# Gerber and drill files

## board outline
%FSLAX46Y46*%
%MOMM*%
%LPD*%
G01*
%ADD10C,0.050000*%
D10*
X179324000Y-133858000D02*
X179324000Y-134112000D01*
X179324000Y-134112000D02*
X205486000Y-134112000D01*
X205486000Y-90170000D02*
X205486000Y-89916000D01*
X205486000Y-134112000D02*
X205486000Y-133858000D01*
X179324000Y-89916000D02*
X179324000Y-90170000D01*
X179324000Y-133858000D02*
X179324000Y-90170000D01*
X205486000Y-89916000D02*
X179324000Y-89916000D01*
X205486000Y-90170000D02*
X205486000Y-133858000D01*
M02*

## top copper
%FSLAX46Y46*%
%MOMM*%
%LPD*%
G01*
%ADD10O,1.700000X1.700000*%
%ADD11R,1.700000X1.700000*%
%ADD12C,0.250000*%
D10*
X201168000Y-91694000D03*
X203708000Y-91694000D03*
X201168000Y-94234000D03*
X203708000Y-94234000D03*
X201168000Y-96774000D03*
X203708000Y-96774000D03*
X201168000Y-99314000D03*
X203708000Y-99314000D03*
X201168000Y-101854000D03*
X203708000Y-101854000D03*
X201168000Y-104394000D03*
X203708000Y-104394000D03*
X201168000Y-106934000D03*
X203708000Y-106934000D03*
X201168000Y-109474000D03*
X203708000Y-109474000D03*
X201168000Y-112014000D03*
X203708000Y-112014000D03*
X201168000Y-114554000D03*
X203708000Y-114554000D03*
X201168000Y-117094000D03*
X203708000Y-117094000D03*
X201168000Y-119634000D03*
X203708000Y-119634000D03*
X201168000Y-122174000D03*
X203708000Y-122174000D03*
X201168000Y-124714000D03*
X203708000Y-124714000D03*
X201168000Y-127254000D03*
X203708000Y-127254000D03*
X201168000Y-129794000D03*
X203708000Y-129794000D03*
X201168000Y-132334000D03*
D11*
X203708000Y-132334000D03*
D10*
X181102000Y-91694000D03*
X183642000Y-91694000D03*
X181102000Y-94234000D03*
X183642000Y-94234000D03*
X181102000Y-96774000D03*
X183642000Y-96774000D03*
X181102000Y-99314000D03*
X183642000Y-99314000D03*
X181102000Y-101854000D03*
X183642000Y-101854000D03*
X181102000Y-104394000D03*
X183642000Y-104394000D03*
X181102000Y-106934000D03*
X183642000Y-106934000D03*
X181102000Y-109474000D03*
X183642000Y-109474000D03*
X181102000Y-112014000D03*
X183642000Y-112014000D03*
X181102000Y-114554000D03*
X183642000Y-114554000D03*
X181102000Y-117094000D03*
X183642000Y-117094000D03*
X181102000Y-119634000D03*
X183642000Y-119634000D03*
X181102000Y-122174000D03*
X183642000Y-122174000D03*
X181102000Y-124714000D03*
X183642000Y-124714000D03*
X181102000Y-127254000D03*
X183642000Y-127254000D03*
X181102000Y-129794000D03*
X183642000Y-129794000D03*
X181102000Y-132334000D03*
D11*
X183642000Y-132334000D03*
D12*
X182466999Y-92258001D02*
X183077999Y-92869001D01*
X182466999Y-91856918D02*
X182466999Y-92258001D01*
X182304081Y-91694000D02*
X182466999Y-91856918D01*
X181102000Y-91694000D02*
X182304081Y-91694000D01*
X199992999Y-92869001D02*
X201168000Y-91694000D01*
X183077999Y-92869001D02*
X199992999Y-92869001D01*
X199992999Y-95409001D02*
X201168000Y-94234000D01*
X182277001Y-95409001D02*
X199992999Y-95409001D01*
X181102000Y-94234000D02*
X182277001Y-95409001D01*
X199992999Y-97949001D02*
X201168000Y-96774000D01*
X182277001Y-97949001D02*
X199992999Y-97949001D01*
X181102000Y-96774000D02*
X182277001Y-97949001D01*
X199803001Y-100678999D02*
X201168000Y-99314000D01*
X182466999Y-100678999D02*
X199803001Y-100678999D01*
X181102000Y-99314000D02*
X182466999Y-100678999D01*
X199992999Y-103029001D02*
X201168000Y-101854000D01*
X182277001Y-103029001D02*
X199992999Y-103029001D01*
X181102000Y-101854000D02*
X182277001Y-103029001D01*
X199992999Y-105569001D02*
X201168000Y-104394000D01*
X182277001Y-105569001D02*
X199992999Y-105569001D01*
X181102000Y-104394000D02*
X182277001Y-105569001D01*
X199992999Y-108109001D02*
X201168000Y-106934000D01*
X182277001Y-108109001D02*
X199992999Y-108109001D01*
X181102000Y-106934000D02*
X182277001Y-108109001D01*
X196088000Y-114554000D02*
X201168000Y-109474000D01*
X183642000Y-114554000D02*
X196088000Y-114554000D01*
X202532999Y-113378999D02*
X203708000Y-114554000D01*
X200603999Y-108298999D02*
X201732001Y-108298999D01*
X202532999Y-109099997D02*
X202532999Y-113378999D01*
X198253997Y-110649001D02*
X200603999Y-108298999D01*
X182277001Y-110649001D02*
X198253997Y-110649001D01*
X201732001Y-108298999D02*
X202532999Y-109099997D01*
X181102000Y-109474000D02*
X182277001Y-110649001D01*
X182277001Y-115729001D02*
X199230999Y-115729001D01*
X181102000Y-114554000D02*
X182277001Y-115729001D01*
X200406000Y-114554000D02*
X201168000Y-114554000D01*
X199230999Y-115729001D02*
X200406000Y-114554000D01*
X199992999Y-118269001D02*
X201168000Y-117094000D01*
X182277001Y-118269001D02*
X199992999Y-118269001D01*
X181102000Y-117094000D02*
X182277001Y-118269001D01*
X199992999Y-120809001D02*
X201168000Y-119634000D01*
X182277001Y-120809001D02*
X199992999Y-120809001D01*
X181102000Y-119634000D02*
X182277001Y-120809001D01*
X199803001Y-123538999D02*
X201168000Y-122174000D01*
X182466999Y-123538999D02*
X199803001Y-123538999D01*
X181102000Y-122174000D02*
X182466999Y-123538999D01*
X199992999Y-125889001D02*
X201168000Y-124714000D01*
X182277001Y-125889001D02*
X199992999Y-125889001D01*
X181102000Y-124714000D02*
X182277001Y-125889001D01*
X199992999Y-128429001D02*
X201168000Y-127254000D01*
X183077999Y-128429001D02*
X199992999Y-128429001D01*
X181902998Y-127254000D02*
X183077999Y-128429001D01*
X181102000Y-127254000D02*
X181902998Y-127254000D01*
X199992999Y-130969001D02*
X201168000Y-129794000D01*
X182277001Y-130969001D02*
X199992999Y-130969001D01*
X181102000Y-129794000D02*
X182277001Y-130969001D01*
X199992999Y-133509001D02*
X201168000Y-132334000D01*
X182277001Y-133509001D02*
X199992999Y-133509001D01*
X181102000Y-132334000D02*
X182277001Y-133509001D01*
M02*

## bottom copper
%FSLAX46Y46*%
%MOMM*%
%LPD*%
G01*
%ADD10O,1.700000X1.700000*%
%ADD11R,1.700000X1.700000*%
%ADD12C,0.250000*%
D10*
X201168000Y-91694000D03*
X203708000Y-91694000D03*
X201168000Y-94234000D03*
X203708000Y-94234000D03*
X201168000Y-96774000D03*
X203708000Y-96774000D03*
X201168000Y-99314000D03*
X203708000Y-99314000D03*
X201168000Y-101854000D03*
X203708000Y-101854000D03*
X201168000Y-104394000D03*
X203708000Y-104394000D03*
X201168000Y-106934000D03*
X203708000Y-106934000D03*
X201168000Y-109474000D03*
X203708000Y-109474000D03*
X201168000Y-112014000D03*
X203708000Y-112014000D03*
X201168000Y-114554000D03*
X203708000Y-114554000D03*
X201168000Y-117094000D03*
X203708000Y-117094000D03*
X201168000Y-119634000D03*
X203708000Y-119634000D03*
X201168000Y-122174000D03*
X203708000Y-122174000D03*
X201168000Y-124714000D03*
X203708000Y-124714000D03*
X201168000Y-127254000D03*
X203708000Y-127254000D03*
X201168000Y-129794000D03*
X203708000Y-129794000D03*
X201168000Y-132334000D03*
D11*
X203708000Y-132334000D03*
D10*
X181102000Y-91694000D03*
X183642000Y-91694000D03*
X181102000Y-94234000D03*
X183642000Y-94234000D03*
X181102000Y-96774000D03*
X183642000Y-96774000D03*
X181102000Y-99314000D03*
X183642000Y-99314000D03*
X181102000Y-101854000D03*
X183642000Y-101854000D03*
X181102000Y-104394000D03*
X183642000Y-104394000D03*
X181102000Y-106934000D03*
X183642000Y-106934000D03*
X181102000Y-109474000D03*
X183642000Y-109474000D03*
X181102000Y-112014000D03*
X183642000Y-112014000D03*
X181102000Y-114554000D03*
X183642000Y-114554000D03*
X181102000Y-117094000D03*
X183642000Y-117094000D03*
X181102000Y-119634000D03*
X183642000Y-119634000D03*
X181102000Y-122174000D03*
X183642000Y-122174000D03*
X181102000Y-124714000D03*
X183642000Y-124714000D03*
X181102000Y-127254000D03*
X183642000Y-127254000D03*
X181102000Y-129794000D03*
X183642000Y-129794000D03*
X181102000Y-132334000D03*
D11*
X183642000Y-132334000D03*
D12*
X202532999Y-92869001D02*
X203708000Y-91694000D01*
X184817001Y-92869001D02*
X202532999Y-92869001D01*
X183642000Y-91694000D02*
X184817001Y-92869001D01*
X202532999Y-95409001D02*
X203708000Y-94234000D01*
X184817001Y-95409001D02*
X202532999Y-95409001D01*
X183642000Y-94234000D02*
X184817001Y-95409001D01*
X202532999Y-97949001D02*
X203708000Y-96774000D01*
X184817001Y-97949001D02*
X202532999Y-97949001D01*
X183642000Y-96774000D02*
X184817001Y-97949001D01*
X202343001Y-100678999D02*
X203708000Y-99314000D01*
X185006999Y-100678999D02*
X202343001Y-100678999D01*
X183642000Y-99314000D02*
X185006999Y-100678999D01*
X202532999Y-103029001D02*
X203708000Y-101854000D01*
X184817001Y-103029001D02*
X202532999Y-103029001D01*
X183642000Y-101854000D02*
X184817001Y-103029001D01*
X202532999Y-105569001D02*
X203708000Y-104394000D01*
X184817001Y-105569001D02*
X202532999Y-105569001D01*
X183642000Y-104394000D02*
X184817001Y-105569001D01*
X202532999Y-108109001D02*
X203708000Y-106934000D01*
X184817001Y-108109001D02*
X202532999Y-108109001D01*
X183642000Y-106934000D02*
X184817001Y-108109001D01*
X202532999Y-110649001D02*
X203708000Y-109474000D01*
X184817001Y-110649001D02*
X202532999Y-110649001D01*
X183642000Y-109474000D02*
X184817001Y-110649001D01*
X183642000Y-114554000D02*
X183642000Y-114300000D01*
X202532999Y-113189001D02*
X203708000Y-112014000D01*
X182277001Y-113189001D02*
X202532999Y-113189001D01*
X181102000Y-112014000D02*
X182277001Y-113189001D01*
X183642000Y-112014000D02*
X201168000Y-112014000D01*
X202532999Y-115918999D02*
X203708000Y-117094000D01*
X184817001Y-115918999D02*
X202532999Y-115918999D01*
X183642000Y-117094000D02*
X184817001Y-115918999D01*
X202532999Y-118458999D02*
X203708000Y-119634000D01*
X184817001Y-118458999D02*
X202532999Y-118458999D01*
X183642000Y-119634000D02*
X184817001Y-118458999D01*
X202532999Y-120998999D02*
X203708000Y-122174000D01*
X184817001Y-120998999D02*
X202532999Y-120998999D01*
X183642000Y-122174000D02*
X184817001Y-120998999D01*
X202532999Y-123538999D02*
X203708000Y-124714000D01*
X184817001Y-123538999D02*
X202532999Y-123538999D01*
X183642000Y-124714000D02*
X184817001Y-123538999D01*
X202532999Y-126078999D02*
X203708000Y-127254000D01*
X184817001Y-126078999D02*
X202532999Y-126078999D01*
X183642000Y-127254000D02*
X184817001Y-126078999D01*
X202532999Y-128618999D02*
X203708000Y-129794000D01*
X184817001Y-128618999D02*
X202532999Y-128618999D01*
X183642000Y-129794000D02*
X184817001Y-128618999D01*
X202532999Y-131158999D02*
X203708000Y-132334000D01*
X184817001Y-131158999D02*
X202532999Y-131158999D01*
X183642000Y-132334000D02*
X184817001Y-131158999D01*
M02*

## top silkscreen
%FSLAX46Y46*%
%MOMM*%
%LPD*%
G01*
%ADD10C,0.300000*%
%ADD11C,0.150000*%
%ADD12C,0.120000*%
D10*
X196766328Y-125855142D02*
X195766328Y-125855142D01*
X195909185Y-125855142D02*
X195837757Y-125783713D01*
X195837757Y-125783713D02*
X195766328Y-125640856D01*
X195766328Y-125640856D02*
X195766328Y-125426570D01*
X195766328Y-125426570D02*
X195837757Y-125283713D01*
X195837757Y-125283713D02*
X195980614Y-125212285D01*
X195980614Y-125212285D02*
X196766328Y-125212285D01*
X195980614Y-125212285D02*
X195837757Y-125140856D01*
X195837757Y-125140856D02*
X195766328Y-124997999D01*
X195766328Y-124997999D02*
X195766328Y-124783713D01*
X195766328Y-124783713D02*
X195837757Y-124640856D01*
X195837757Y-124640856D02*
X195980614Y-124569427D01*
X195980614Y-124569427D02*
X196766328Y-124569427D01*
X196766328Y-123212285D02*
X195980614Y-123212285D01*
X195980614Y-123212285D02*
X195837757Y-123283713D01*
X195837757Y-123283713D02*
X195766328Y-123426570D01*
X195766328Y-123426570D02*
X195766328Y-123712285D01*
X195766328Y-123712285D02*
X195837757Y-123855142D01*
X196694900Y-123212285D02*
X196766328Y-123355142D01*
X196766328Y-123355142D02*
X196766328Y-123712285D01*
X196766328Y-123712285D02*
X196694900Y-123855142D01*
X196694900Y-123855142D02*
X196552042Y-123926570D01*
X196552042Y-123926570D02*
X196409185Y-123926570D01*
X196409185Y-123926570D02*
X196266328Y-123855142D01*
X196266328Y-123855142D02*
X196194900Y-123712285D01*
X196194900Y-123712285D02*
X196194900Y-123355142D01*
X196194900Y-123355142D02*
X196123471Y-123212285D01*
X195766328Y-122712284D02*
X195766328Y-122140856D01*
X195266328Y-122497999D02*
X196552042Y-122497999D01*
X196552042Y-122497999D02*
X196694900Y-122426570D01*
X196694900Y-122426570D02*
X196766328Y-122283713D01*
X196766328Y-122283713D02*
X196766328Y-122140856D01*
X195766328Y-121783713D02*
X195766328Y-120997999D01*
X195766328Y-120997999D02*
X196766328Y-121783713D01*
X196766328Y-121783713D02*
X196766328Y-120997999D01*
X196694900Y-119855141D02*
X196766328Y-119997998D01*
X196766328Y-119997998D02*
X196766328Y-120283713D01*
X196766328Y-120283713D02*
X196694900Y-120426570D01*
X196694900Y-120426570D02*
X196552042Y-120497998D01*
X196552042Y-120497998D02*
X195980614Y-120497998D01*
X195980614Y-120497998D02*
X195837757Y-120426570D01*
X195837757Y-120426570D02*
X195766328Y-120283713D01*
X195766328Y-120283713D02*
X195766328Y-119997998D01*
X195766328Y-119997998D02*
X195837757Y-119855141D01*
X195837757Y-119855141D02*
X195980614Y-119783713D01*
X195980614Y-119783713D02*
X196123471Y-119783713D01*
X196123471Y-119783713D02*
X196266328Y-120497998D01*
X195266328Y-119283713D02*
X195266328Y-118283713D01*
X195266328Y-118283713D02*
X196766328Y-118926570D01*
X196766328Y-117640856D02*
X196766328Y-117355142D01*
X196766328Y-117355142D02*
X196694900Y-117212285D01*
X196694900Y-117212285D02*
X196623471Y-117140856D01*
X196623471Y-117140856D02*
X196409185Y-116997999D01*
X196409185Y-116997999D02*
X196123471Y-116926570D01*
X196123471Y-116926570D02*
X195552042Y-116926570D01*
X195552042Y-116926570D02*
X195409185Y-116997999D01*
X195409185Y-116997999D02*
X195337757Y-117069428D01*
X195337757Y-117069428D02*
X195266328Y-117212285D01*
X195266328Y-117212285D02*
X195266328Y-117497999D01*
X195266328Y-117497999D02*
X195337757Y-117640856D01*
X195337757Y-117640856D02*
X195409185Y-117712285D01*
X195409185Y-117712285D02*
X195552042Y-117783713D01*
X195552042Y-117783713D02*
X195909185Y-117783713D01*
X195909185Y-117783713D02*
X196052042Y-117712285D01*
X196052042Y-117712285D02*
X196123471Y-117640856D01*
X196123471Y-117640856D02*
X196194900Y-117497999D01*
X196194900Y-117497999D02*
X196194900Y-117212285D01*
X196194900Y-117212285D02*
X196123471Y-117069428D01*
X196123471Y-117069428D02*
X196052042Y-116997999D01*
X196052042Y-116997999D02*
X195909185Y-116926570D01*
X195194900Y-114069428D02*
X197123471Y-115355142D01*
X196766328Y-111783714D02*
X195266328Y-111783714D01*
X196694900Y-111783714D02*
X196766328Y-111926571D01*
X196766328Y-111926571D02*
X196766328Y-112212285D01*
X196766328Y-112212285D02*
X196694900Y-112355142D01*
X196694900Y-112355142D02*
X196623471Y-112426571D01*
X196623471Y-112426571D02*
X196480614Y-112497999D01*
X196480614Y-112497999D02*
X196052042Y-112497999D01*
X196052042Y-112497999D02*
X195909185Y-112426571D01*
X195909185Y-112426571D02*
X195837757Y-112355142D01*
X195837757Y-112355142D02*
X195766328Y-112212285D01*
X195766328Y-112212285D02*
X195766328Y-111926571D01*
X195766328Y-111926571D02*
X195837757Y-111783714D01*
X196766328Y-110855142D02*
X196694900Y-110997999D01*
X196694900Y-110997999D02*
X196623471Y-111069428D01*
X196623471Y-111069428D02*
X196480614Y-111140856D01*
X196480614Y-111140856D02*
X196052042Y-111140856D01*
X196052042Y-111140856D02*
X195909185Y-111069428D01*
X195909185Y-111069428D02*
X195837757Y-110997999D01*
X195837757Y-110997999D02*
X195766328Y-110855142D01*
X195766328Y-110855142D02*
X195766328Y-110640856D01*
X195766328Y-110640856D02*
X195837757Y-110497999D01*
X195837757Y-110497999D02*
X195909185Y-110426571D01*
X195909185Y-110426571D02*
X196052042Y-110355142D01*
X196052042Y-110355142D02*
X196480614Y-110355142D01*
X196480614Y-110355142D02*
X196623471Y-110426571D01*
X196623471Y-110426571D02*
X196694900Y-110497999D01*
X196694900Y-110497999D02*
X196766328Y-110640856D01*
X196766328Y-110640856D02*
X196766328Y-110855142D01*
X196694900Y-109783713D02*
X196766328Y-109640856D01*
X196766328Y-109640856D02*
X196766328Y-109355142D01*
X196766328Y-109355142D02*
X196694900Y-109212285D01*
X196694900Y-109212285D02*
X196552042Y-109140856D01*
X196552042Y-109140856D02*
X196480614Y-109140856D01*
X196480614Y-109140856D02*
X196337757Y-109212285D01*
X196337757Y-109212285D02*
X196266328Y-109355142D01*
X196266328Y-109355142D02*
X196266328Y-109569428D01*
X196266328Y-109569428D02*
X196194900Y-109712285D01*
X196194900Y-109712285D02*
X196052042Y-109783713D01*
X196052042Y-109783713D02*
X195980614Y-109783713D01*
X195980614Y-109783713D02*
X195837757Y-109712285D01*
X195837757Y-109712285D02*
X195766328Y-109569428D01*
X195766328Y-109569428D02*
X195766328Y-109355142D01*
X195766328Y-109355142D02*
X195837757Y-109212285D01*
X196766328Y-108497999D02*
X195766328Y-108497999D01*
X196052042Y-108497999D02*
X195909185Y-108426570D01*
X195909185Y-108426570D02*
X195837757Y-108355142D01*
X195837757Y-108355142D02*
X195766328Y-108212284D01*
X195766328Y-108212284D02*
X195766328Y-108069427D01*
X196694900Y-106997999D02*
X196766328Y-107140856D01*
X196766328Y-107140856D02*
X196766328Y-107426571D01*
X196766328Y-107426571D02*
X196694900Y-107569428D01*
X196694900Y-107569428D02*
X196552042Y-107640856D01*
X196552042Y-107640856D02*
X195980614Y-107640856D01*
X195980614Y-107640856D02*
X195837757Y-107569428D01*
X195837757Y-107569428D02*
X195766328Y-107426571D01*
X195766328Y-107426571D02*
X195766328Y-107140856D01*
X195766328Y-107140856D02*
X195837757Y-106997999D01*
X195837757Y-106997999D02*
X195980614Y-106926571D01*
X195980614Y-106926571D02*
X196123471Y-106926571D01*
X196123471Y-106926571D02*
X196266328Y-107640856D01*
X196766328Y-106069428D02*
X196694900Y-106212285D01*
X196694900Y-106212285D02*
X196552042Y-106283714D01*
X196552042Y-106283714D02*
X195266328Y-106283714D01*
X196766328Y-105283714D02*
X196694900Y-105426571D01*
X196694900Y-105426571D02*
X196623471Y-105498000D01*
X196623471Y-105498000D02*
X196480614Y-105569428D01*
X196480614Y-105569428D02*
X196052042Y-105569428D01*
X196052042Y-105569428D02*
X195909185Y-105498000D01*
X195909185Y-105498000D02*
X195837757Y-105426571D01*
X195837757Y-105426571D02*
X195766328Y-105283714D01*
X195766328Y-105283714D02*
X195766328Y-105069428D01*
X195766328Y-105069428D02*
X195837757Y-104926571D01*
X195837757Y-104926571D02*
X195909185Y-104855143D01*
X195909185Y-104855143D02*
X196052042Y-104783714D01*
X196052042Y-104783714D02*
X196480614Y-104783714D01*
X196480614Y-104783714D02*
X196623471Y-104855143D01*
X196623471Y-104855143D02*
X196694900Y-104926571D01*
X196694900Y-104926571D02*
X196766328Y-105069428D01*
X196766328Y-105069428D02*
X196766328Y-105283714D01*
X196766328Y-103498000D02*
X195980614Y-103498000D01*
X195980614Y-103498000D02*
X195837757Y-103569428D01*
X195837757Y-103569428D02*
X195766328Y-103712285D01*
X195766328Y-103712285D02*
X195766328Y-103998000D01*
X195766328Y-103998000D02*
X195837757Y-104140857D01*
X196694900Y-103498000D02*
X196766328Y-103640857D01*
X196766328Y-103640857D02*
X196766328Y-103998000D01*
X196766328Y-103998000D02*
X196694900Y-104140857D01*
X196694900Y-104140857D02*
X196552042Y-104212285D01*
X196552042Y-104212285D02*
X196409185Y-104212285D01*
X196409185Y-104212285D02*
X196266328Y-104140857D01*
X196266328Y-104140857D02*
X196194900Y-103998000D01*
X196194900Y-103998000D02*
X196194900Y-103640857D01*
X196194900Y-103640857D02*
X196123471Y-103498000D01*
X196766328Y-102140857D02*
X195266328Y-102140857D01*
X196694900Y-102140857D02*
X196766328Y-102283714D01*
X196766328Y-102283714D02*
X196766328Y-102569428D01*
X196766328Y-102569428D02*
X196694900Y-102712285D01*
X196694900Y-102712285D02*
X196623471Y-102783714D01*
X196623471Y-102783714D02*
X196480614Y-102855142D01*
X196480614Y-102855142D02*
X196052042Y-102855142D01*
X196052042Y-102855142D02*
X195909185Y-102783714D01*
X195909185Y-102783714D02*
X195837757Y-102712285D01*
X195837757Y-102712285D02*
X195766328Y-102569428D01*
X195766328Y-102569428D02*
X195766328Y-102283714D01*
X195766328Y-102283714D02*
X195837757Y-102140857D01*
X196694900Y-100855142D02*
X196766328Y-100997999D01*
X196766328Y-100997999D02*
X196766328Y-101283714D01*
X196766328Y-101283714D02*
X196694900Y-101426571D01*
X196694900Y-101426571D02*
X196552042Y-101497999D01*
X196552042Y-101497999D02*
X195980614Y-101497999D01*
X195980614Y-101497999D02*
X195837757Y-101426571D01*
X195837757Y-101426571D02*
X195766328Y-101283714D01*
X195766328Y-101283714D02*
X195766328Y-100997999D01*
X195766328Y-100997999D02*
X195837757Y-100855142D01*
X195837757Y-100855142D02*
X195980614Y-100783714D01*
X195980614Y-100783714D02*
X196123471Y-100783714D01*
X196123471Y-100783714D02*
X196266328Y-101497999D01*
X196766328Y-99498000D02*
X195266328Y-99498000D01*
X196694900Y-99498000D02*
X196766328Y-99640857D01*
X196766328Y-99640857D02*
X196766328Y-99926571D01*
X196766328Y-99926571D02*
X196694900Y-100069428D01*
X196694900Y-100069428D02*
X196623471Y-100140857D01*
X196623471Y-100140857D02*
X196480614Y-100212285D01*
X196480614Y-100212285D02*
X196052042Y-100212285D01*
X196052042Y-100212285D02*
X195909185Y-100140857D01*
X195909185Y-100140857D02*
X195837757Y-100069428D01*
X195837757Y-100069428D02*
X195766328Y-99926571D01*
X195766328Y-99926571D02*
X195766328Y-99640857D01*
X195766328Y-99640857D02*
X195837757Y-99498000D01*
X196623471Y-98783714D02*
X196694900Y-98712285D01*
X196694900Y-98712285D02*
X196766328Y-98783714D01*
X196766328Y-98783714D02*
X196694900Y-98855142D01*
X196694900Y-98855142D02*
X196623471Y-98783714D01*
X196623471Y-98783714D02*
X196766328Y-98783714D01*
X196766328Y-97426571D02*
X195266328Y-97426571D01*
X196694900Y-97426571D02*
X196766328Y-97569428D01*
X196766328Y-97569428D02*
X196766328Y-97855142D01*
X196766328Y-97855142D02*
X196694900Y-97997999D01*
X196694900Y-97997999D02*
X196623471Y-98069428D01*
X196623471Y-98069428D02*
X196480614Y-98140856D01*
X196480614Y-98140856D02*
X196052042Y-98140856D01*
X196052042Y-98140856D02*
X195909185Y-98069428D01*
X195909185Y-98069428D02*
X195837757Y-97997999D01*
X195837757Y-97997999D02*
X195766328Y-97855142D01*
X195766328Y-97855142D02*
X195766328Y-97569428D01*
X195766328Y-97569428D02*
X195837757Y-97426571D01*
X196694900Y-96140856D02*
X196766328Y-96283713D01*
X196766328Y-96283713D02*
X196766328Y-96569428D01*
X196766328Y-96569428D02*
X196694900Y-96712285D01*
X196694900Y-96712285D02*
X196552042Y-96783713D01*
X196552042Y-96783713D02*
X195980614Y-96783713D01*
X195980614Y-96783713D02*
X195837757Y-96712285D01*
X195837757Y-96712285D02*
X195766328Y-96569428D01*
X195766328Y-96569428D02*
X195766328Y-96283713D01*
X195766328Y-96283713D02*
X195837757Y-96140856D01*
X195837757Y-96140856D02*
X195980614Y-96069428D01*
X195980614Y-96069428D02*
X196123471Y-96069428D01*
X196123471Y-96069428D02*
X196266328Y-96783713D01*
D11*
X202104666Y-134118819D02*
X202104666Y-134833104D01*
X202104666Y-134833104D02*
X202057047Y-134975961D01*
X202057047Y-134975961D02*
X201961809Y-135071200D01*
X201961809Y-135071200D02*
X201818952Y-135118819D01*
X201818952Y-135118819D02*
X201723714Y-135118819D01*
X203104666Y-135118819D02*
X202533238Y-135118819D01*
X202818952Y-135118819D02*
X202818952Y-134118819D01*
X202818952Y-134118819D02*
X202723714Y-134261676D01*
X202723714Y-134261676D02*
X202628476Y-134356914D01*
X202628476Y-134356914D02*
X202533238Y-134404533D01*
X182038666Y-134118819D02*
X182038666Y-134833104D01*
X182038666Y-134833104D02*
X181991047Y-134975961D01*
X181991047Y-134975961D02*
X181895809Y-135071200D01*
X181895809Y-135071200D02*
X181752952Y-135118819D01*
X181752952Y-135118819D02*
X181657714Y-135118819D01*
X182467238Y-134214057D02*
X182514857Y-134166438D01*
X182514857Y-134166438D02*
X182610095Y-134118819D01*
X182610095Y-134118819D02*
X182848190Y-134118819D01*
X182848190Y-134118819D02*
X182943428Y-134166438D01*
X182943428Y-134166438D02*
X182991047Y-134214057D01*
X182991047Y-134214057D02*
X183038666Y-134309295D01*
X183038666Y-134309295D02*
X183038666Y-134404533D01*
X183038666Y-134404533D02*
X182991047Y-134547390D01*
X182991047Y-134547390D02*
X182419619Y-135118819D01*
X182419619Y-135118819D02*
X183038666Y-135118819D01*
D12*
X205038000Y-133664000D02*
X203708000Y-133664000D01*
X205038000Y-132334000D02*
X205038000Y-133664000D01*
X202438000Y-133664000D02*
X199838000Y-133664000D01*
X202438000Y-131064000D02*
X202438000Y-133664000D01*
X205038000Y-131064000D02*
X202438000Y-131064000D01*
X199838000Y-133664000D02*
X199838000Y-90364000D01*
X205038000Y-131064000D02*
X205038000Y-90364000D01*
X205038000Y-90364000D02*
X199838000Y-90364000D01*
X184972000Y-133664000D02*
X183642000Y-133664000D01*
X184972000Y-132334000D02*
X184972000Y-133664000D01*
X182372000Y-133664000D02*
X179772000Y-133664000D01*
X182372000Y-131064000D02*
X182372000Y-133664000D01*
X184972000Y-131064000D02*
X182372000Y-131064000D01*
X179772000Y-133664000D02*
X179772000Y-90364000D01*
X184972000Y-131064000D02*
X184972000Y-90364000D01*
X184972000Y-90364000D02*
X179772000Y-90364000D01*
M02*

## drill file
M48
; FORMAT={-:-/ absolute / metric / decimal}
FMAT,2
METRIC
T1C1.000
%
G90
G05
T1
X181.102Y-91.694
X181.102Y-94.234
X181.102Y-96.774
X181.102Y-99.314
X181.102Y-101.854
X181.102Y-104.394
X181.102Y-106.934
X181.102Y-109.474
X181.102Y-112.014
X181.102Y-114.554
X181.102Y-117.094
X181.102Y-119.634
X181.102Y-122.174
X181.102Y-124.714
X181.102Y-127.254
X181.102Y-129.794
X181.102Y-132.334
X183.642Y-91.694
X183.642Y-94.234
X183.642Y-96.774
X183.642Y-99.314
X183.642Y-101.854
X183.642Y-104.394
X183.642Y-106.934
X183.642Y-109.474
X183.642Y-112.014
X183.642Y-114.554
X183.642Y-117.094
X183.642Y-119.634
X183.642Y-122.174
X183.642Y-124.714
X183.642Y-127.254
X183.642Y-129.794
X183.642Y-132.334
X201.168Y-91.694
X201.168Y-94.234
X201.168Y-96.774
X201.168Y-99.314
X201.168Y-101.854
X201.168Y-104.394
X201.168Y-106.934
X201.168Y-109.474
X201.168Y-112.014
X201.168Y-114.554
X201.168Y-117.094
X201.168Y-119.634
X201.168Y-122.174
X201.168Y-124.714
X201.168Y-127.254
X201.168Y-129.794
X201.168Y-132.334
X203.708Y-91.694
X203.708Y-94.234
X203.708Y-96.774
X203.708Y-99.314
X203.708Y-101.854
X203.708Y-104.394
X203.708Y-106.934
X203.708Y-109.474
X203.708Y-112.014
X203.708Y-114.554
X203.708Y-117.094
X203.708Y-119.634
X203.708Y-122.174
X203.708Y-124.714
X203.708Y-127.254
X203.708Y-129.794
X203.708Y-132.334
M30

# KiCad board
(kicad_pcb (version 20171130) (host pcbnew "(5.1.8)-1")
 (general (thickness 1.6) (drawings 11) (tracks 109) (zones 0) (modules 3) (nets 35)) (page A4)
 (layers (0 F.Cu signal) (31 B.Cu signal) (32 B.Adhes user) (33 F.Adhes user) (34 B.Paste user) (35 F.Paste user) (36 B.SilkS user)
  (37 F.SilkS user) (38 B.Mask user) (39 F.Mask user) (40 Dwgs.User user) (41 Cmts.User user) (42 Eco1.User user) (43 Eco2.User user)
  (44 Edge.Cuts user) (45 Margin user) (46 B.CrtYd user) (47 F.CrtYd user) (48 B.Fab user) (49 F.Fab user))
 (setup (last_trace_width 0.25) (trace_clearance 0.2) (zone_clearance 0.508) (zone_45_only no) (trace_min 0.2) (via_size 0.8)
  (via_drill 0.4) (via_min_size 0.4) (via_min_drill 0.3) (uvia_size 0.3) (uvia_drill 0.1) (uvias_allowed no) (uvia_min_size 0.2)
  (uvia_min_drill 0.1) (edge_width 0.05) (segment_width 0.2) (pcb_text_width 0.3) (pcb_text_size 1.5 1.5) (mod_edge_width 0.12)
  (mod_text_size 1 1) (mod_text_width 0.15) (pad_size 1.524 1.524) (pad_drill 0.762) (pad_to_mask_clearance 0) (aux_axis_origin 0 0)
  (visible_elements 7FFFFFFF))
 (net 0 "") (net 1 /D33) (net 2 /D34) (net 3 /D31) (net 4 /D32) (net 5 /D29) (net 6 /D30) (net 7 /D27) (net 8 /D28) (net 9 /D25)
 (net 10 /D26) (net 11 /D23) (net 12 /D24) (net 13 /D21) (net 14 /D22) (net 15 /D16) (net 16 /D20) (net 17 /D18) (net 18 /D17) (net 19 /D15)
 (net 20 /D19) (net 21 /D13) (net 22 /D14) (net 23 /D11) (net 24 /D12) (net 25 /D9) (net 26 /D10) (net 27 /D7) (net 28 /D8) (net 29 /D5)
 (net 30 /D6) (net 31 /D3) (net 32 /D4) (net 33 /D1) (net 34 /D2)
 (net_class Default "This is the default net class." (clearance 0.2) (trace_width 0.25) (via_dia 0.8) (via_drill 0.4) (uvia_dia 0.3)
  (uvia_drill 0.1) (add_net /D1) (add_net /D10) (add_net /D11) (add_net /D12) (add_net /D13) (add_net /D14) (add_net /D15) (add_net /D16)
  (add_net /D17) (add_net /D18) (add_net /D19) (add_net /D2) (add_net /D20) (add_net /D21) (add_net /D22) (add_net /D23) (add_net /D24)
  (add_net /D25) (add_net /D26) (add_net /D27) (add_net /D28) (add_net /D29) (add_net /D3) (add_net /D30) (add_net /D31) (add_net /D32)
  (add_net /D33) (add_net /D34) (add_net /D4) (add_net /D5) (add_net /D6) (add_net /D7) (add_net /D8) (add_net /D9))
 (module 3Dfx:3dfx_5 (layer B.Cu) (at 193.294 112.776 270)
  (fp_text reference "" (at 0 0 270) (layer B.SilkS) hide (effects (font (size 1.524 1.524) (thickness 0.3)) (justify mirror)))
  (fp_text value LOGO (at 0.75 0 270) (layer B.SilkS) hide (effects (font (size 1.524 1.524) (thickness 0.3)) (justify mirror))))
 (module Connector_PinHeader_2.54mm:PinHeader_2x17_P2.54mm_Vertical (layer F.Cu) (at 203.708 132.334 180)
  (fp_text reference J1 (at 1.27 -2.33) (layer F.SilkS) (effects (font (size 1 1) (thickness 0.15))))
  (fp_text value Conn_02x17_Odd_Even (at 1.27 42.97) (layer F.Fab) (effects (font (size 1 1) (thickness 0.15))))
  (fp_line (start -1.33 -1.33) (end 0 -1.33) (layer F.SilkS) (width 0.12))
  (fp_line (start -1.33 0) (end -1.33 -1.33) (layer F.SilkS) (width 0.12))
  (fp_line (start 1.27 -1.33) (end 3.87 -1.33) (layer F.SilkS) (width 0.12))
  (fp_line (start 1.27 1.27) (end 1.27 -1.33) (layer F.SilkS) (width 0.12))
  (fp_line (start -1.33 1.27) (end 1.27 1.27) (layer F.SilkS) (width 0.12))
  (fp_line (start 3.87 -1.33) (end 3.87 41.97) (layer F.SilkS) (width 0.12))
  (fp_line (start -1.33 1.27) (end -1.33 41.97) (layer F.SilkS) (width 0.12))
  (fp_line (start -1.33 41.97) (end 3.87 41.97) (layer F.SilkS) (width 0.12))
  (pad 34 thru_hole oval (at 2.54 40.64 180) (size 1.7 1.7) (drill 1) (layers *.Cu *.Mask) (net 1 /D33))
  (pad 33 thru_hole oval (at 0 40.64 180) (size 1.7 1.7) (drill 1) (layers *.Cu *.Mask) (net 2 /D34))
  (pad 32 thru_hole oval (at 2.54 38.1 180) (size 1.7 1.7) (drill 1) (layers *.Cu *.Mask) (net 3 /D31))
  (pad 31 thru_hole oval (at 0 38.1 180) (size 1.7 1.7) (drill 1) (layers *.Cu *.Mask) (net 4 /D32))
  (pad 30 thru_hole oval (at 2.54 35.56 180) (size 1.7 1.7) (drill 1) (layers *.Cu *.Mask) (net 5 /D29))
  (pad 29 thru_hole oval (at 0 35.56 180) (size 1.7 1.7) (drill 1) (layers *.Cu *.Mask) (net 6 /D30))
  (pad 28 thru_hole oval (at 2.54 33.02 180) (size 1.7 1.7) (drill 1) (layers *.Cu *.Mask) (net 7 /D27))
  (pad 27 thru_hole oval (at 0 33.02 180) (size 1.7 1.7) (drill 1) (layers *.Cu *.Mask) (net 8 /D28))
  (pad 26 thru_hole oval (at 2.54 30.48 180) (size 1.7 1.7) (drill 1) (layers *.Cu *.Mask) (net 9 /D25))
  (pad 25 thru_hole oval (at 0 30.48 180) (size 1.7 1.7) (drill 1) (layers *.Cu *.Mask) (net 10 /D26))
  (pad 24 thru_hole oval (at 2.54 27.94 180) (size 1.7 1.7) (drill 1) (layers *.Cu *.Mask) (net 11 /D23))
  (pad 23 thru_hole oval (at 0 27.94 180) (size 1.7 1.7) (drill 1) (layers *.Cu *.Mask) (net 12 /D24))
  (pad 22 thru_hole oval (at 2.54 25.4 180) (size 1.7 1.7) (drill 1) (layers *.Cu *.Mask) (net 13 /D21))
  (pad 21 thru_hole oval (at 0 25.4 180) (size 1.7 1.7) (drill 1) (layers *.Cu *.Mask) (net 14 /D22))
  (pad 20 thru_hole oval (at 2.54 22.86 180) (size 1.7 1.7) (drill 1) (layers *.Cu *.Mask) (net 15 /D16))
  (pad 19 thru_hole oval (at 0 22.86 180) (size 1.7 1.7) (drill 1) (layers *.Cu *.Mask) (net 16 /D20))
  (pad 18 thru_hole oval (at 2.54 20.32 180) (size 1.7 1.7) (drill 1) (layers *.Cu *.Mask) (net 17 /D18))
  (pad 17 thru_hole oval (at 0 20.32 180) (size 1.7 1.7) (drill 1) (layers *.Cu *.Mask) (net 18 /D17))
  (pad 16 thru_hole oval (at 2.54 17.78 180) (size 1.7 1.7) (drill 1) (layers *.Cu *.Mask) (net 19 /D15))
  (pad 15 thru_hole oval (at 0 17.78 180) (size 1.7 1.7) (drill 1) (layers *.Cu *.Mask) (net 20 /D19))
  (pad 14 thru_hole oval (at 2.54 15.24 180) (size 1.7 1.7) (drill 1) (layers *.Cu *.Mask) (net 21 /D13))
  (pad 13 thru_hole oval (at 0 15.24 180) (size 1.7 1.7) (drill 1) (layers *.Cu *.Mask) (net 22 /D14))
  (pad 12 thru_hole oval (at 2.54 12.7 180) (size 1.7 1.7) (drill 1) (layers *.Cu *.Mask) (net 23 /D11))
  (pad 11 thru_hole oval (at 0 12.7 180) (size 1.7 1.7) (drill 1) (layers *.Cu *.Mask) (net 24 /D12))
  (pad 10 thru_hole oval (at 2.54 10.16 180) (size 1.7 1.7) (drill 1) (layers *.Cu *.Mask) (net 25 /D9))
  (pad 9 thru_hole oval (at 0 10.16 180) (size 1.7 1.7) (drill 1) (layers *.Cu *.Mask) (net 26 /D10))
  (pad 8 thru_hole oval (at 2.54 7.62 180) (size 1.7 1.7) (drill 1) (layers *.Cu *.Mask) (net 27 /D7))
  (pad 7 thru_hole oval (at 0 7.62 180) (size 1.7 1.7) (drill 1) (layers *.Cu *.Mask) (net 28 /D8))
  (pad 6 thru_hole oval (at 2.54 5.08 180) (size 1.7 1.7) (drill 1) (layers *.Cu *.Mask) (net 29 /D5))
  (pad 5 thru_hole oval (at 0 5.08 180) (size 1.7 1.7) (drill 1) (layers *.Cu *.Mask) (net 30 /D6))
  (pad 4 thru_hole oval (at 2.54 2.54 180) (size 1.7 1.7) (drill 1) (layers *.Cu *.Mask) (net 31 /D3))
  (pad 3 thru_hole oval (at 0 2.54 180) (size 1.7 1.7) (drill 1) (layers *.Cu *.Mask) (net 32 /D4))
  (pad 2 thru_hole oval (at 2.54 0 180) (size 1.7 1.7) (drill 1) (layers *.Cu *.Mask) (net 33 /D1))
  (pad 1 thru_hole rect (at 0 0 180) (size 1.7 1.7) (drill 1) (layers *.Cu *.Mask) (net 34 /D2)))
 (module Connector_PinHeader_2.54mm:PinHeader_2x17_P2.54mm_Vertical (layer F.Cu) (at 183.642 132.334 180)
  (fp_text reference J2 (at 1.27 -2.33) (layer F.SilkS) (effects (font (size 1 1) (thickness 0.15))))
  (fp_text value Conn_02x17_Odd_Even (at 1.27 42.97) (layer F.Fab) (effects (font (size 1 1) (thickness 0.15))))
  (fp_line (start -1.33 -1.33) (end 0 -1.33) (layer F.SilkS) (width 0.12))
  (fp_line (start -1.33 0) (end -1.33 -1.33) (layer F.SilkS) (width 0.12))
  (fp_line (start 1.27 -1.33) (end 3.87 -1.33) (layer F.SilkS) (width 0.12))
  (fp_line (start 1.27 1.27) (end 1.27 -1.33) (layer F.SilkS) (width 0.12))
  (fp_line (start -1.33 1.27) (end 1.27 1.27) (layer F.SilkS) (width 0.12))
  (fp_line (start 3.87 -1.33) (end 3.87 41.97) (layer F.SilkS) (width 0.12))
  (fp_line (start -1.33 1.27) (end -1.33 41.97) (layer F.SilkS) (width 0.12))
  (fp_line (start -1.33 41.97) (end 3.87 41.97) (layer F.SilkS) (width 0.12))
  (pad 34 thru_hole oval (at 2.54 40.64 180) (size 1.7 1.7) (drill 1) (layers *.Cu *.Mask) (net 1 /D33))
  (pad 33 thru_hole oval (at 0 40.64 180) (size 1.7 1.7) (drill 1) (layers *.Cu *.Mask) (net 2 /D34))
  (pad 32 thru_hole oval (at 2.54 38.1 180) (size 1.7 1.7) (drill 1) (layers *.Cu *.Mask) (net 3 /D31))
  (pad 31 thru_hole oval (at 0 38.1 180) (size 1.7 1.7) (drill 1) (layers *.Cu *.Mask) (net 4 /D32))
  (pad 30 thru_hole oval (at 2.54 35.56 180) (size 1.7 1.7) (drill 1) (layers *.Cu *.Mask) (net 5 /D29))
  (pad 29 thru_hole oval (at 0 35.56 180) (size 1.7 1.7) (drill 1) (layers *.Cu *.Mask) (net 6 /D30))
  (pad 28 thru_hole oval (at 2.54 33.02 180) (size 1.7 1.7) (drill 1) (layers *.Cu *.Mask) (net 7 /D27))
  (pad 27 thru_hole oval (at 0 33.02 180) (size 1.7 1.7) (drill 1) (layers *.Cu *.Mask) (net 8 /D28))
  (pad 26 thru_hole oval (at 2.54 30.48 180) (size 1.7 1.7) (drill 1) (layers *.Cu *.Mask) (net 9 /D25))
  (pad 25 thru_hole oval (at 0 30.48 180) (size 1.7 1.7) (drill 1) (layers *.Cu *.Mask) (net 10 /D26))
  (pad 24 thru_hole oval (at 2.54 27.94 180) (size 1.7 1.7) (drill 1) (layers *.Cu *.Mask) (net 11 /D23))
  (pad 23 thru_hole oval (at 0 27.94 180) (size 1.7 1.7) (drill 1) (layers *.Cu *.Mask) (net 12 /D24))
  (pad 22 thru_hole oval (at 2.54 25.4 180) (size 1.7 1.7) (drill 1) (layers *.Cu *.Mask) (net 13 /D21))
  (pad 21 thru_hole oval (at 0 25.4 180) (size 1.7 1.7) (drill 1) (layers *.Cu *.Mask) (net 14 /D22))
  (pad 20 thru_hole oval (at 2.54 22.86 180) (size 1.7 1.7) (drill 1) (layers *.Cu *.Mask) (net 20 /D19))
  (pad 19 thru_hole oval (at 0 22.86 180) (size 1.7 1.7) (drill 1) (layers *.Cu *.Mask) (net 16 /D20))
  (pad 18 thru_hole oval (at 2.54 20.32 180) (size 1.7 1.7) (drill 1) (layers *.Cu *.Mask) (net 18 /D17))
  (pad 17 thru_hole oval (at 0 20.32 180) (size 1.7 1.7) (drill 1) (layers *.Cu *.Mask) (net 17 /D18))
  (pad 16 thru_hole oval (at 2.54 17.78 180) (size 1.7 1.7) (drill 1) (layers *.Cu *.Mask) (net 19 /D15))
  (pad 15 thru_hole oval (at 0 17.78 180) (size 1.7 1.7) (drill 1) (layers *.Cu *.Mask) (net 15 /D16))
  (pad 14 thru_hole oval (at 2.54 15.24 180) (size 1.7 1.7) (drill 1) (layers *.Cu *.Mask) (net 21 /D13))
  (pad 13 thru_hole oval (at 0 15.24 180) (size 1.7 1.7) (drill 1) (layers *.Cu *.Mask) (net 22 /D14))
  (pad 12 thru_hole oval (at 2.54 12.7 180) (size 1.7 1.7) (drill 1) (layers *.Cu *.Mask) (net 23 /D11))
  (pad 11 thru_hole oval (at 0 12.7 180) (size 1.7 1.7) (drill 1) (layers *.Cu *.Mask) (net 24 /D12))
  (pad 10 thru_hole oval (at 2.54 10.16 180) (size 1.7 1.7) (drill 1) (layers *.Cu *.Mask) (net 25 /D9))
  (pad 9 thru_hole oval (at 0 10.16 180) (size 1.7 1.7) (drill 1) (layers *.Cu *.Mask) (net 26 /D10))
  (pad 8 thru_hole oval (at 2.54 7.62 180) (size 1.7 1.7) (drill 1) (layers *.Cu *.Mask) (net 27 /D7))
  (pad 7 thru_hole oval (at 0 7.62 180) (size 1.7 1.7) (drill 1) (layers *.Cu *.Mask) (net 28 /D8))
  (pad 6 thru_hole oval (at 2.54 5.08 180) (size 1.7 1.7) (drill 1) (layers *.Cu *.Mask) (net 29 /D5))
  (pad 5 thru_hole oval (at 0 5.08 180) (size 1.7 1.7) (drill 1) (layers *.Cu *.Mask) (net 30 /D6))
  (pad 4 thru_hole oval (at 2.54 2.54 180) (size 1.7 1.7) (drill 1) (layers *.Cu *.Mask) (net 31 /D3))
  (pad 3 thru_hole oval (at 0 2.54 180) (size 1.7 1.7) (drill 1) (layers *.Cu *.Mask) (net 32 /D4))
  (pad 2 thru_hole oval (at 2.54 0 180) (size 1.7 1.7) (drill 1) (layers *.Cu *.Mask) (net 33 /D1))
  (pad 1 thru_hole rect (at 0 0 180) (size 1.7 1.7) (drill 1) (layers *.Cu *.Mask) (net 34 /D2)))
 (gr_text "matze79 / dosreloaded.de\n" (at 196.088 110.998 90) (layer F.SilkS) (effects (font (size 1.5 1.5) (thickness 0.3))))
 (gr_line (start 179.324 133.858) (end 179.324 134.112) (layer Edge.Cuts) (width 0.05))
 (gr_line (start 179.324 134.112) (end 205.486 134.112) (layer Edge.Cuts) (width 0.05))
 (gr_line (start 205.486 90.17) (end 205.486 89.916) (layer Edge.Cuts) (width 0.05))
 (gr_line (start 205.486 134.112) (end 205.486 133.858) (layer Edge.Cuts) (width 0.05))
 (gr_line (start 179.324 89.916) (end 179.324 90.17) (layer Edge.Cuts) (width 0.05))
 (gr_line (start 179.324 133.858) (end 179.324 90.17) (layer Edge.Cuts) (width 0.05))
 (gr_line (start 205.486 89.916) (end 179.324 89.916) (layer Edge.Cuts) (width 0.05))
 (gr_line (start 205.486 90.17) (end 205.486 133.858) (layer Edge.Cuts) (width 0.05))
 (segment (start 202.532999 92.869001) (end 203.708 91.694) (width 0.25) (layer B.Cu) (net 2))
 (segment (start 184.817001 92.869001) (end 202.532999 92.869001) (width 0.25) (layer B.Cu) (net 2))
 (segment (start 183.642 91.694) (end 184.817001 92.869001) (width 0.25) (layer B.Cu) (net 2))
 (segment (start 182.466999 92.258001) (end 183.077999 92.869001) (width 0.25) (layer F.Cu) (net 1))
 (segment (start 182.466999 91.856918) (end 182.466999 92.258001) (width 0.25) (layer F.Cu) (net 1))
 (segment (start 182.304081 91.694) (end 182.466999 91.856918) (width 0.25) (layer F.Cu) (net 1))
 (segment (start 181.102 91.694) (end 182.304081 91.694) (width 0.25) (layer F.Cu) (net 1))
 (segment (start 199.992999 92.869001) (end 201.168 91.694) (width 0.25) (layer F.Cu) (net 1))
 (segment (start 183.077999 92.869001) (end 199.992999 92.869001) (width 0.25) (layer F.Cu) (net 1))
 (segment (start 202.532999 95.409001) (end 203.708 94.234) (width 0.25) (layer B.Cu) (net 4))
 (segment (start 184.817001 95.409001) (end 202.532999 95.409001) (width 0.25) (layer B.Cu) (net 4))
 (segment (start 183.642 94.234) (end 184.817001 95.409001) (width 0.25) (layer B.Cu) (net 4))
 (segment (start 199.992999 95.409001) (end 201.168 94.234) (width 0.25) (layer F.Cu) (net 3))
 (segment (start 182.277001 95.409001) (end 199.992999 95.409001) (width 0.25) (layer F.Cu) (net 3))
 (segment (start 181.102 94.234) (end 182.277001 95.409001) (width 0.25) (layer F.Cu) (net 3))
 (segment (start 202.532999 97.949001) (end 203.708 96.774) (width 0.25) (layer B.Cu) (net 6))
 (segment (start 184.817001 97.949001) (end 202.532999 97.949001) (width 0.25) (layer B.Cu) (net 6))
 (segment (start 183.642 96.774) (end 184.817001 97.949001) (width 0.25) (layer B.Cu) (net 6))
 (segment (start 199.992999 97.949001) (end 201.168 96.774) (width 0.25) (layer F.Cu) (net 5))
 (segment (start 182.277001 97.949001) (end 199.992999 97.949001) (width 0.25) (layer F.Cu) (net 5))
 (segment (start 181.102 96.774) (end 182.277001 97.949001) (width 0.25) (layer F.Cu) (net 5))
 (segment (start 202.343001 100.678999) (end 203.708 99.314) (width 0.25) (layer B.Cu) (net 8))
 (segment (start 185.006999 100.678999) (end 202.343001 100.678999) (width 0.25) (layer B.Cu) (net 8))
 (segment (start 183.642 99.314) (end 185.006999 100.678999) (width 0.25) (layer B.Cu) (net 8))
 (segment (start 199.803001 100.678999) (end 201.168 99.314) (width 0.25) (layer F.Cu) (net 7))
 (segment (start 182.466999 100.678999) (end 199.803001 100.678999) (width 0.25) (layer F.Cu) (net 7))
 (segment (start 181.102 99.314) (end 182.466999 100.678999) (width 0.25) (layer F.Cu) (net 7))
 (segment (start 202.532999 103.029001) (end 203.708 101.854) (width 0.25) (layer B.Cu) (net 10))
 (segment (start 184.817001 103.029001) (end 202.532999 103.029001) (width 0.25) (layer B.Cu) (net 10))
 (segment (start 183.642 101.854) (end 184.817001 103.029001) (width 0.25) (layer B.Cu) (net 10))
 (segment (start 199.992999 103.029001) (end 201.168 101.854) (width 0.25) (layer F.Cu) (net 9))
 (segment (start 182.277001 103.029001) (end 199.992999 103.029001) (width 0.25) (layer F.Cu) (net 9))
 (segment (start 181.102 101.854) (end 182.277001 103.029001) (width 0.25) (layer F.Cu) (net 9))
 (segment (start 202.532999 105.569001) (end 203.708 104.394) (width 0.25) (layer B.Cu) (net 12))
 (segment (start 184.817001 105.569001) (end 202.532999 105.569001) (width 0.25) (layer B.Cu) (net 12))
 (segment (start 183.642 104.394) (end 184.817001 105.569001) (width 0.25) (layer B.Cu) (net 12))
 (segment (start 199.992999 105.569001) (end 201.168 104.394) (width 0.25) (layer F.Cu) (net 11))
 (segment (start 182.277001 105.569001) (end 199.992999 105.569001) (width 0.25) (layer F.Cu) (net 11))
 (segment (start 181.102 104.394) (end 182.277001 105.569001) (width 0.25) (layer F.Cu) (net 11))
 (segment (start 202.532999 108.109001) (end 203.708 106.934) (width 0.25) (layer B.Cu) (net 14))
 (segment (start 184.817001 108.109001) (end 202.532999 108.109001) (width 0.25) (layer B.Cu) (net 14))
 (segment (start 183.642 106.934) (end 184.817001 108.109001) (width 0.25) (layer B.Cu) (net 14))
 (segment (start 199.992999 108.109001) (end 201.168 106.934) (width 0.25) (layer F.Cu) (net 13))
 (segment (start 182.277001 108.109001) (end 199.992999 108.109001) (width 0.25) (layer F.Cu) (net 13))
 (segment (start 181.102 106.934) (end 182.277001 108.109001) (width 0.25) (layer F.Cu) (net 13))
 (segment (start 202.532999 110.649001) (end 203.708 109.474) (width 0.25) (layer B.Cu) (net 16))
 (segment (start 184.817001 110.649001) (end 202.532999 110.649001) (width 0.25) (layer B.Cu) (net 16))
 (segment (start 183.642 109.474) (end 184.817001 110.649001) (width 0.25) (layer B.Cu) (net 16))
 (segment (start 183.642 114.554) (end 183.642 114.3) (width 0.25) (layer B.Cu) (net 15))
 (segment (start 196.088 114.554) (end 201.168 109.474) (width 0.25) (layer F.Cu) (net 15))
 (segment (start 183.642 114.554) (end 196.088 114.554) (width 0.25) (layer F.Cu) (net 15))
 (segment (start 202.532999 113.189001) (end 203.708 112.014) (width 0.25) (layer B.Cu) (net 18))
 (segment (start 182.277001 113.189001) (end 202.532999 113.189001) (width 0.25) (layer B.Cu) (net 18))
 (segment (start 181.102 112.014) (end 182.277001 113.189001) (width 0.25) (layer B.Cu) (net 18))
 (segment (start 183.642 112.014) (end 201.168 112.014) (width 0.25) (layer B.Cu) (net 17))
 (segment (start 202.532999 113.378999) (end 203.708 114.554) (width 0.25) (layer F.Cu) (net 20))
 (segment (start 200.603999 108.298999) (end 201.732001 108.298999) (width 0.25) (layer F.Cu) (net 20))
 (segment (start 202.532999 109.099997) (end 202.532999 113.378999) (width 0.25) (layer F.Cu) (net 20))
 (segment (start 198.253997 110.649001) (end 200.603999 108.298999) (width 0.25) (layer F.Cu) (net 20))
 (segment (start 182.277001 110.649001) (end 198.253997 110.649001) (width 0.25) (layer F.Cu) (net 20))
 (segment (start 201.732001 108.298999) (end 202.532999 109.099997) (width 0.25) (layer F.Cu) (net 20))
 (segment (start 181.102 109.474) (end 182.277001 110.649001) (width 0.25) (layer F.Cu) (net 20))
 (segment (start 182.277001 115.729001) (end 199.230999 115.729001) (width 0.25) (layer F.Cu) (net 19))
 (segment (start 181.102 114.554) (end 182.277001 115.729001) (width 0.25) (layer F.Cu) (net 19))
 (segment (start 200.406 114.554) (end 201.168 114.554) (width 0.25) (layer F.Cu) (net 19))
 (segment (start 199.230999 115.729001) (end 200.406 114.554) (width 0.25) (layer F.Cu) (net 19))
 (segment (start 202.532999 115.918999) (end 203.708 117.094) (width 0.25) (layer B.Cu) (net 22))
 (segment (start 184.817001 115.918999) (end 202.532999 115.918999) (width 0.25) (layer B.Cu) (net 22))
 (segment (start 183.642 117.094) (end 184.817001 115.918999) (width 0.25) (layer B.Cu) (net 22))
 (segment (start 199.992999 118.269001) (end 201.168 117.094) (width 0.25) (layer F.Cu) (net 21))
 (segment (start 182.277001 118.269001) (end 199.992999 118.269001) (width 0.25) (layer F.Cu) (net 21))
 (segment (start 181.102 117.094) (end 182.277001 118.269001) (width 0.25) (layer F.Cu) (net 21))
 (segment (start 202.532999 118.458999) (end 203.708 119.634) (width 0.25) (layer B.Cu) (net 24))
 (segment (start 184.817001 118.458999) (end 202.532999 118.458999) (width 0.25) (layer B.Cu) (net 24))
 (segment (start 183.642 119.634) (end 184.817001 118.458999) (width 0.25) (layer B.Cu) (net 24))
 (segment (start 199.992999 120.809001) (end 201.168 119.634) (width 0.25) (layer F.Cu) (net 23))
 (segment (start 182.277001 120.809001) (end 199.992999 120.809001) (width 0.25) (layer F.Cu) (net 23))
 (segment (start 181.102 119.634) (end 182.277001 120.809001) (width 0.25) (layer F.Cu) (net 23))
 (segment (start 202.532999 120.998999) (end 203.708 122.174) (width 0.25) (layer B.Cu) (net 26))
 (segment (start 184.817001 120.998999) (end 202.532999 120.998999) (width 0.25) (layer B.Cu) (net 26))
 (segment (start 183.642 122.174) (end 184.817001 120.998999) (width 0.25) (layer B.Cu) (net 26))
 (segment (start 199.803001 123.538999) (end 201.168 122.174) (width 0.25) (layer F.Cu) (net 25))
 (segment (start 182.466999 123.538999) (end 199.803001 123.538999) (width 0.25) (layer F.Cu) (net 25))
 (segment (start 181.102 122.174) (end 182.466999 123.538999) (width 0.25) (layer F.Cu) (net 25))
 (segment (start 202.532999 123.538999) (end 203.708 124.714) (width 0.25) (layer B.Cu) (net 28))
 (segment (start 184.817001 123.538999) (end 202.532999 123.538999) (width 0.25) (layer B.Cu) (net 28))
 (segment (start 183.642 124.714) (end 184.817001 123.538999) (width 0.25) (layer B.Cu) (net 28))
 (segment (start 199.992999 125.889001) (end 201.168 124.714) (width 0.25) (layer F.Cu) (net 27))
 (segment (start 182.277001 125.889001) (end 199.992999 125.889001) (width 0.25) (layer F.Cu) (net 27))
 (segment (start 181.102 124.714) (end 182.277001 125.889001) (width 0.25) (layer F.Cu) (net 27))
 (segment (start 202.532999 126.078999) (end 203.708 127.254) (width 0.25) (layer B.Cu) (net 30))
 (segment (start 184.817001 126.078999) (end 202.532999 126.078999) (width 0.25) (layer B.Cu) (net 30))
 (segment (start 183.642 127.254) (end 184.817001 126.078999) (width 0.25) (layer B.Cu) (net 30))
 (segment (start 199.992999 128.429001) (end 201.168 127.254) (width 0.25) (layer F.Cu) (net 29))
 (segment (start 183.077999 128.429001) (end 199.992999 128.429001) (width 0.25) (layer F.Cu) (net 29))
 (segment (start 181.902998 127.254) (end 183.077999 128.429001) (width 0.25) (layer F.Cu) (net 29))
 (segment (start 181.102 127.254) (end 181.902998 127.254) (width 0.25) (layer F.Cu) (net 29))
 (segment (start 202.532999 128.618999) (end 203.708 129.794) (width 0.25) (layer B.Cu) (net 32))
 (segment (start 184.817001 128.618999) (end 202.532999 128.618999) (width 0.25) (layer B.Cu) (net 32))
 (segment (start 183.642 129.794) (end 184.817001 128.618999) (width 0.25) (layer B.Cu) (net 32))
 (segment (start 199.992999 130.969001) (end 201.168 129.794) (width 0.25) (layer F.Cu) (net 31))
 (segment (start 182.277001 130.969001) (end 199.992999 130.969001) (width 0.25) (layer F.Cu) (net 31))
 (segment (start 181.102 129.794) (end 182.277001 130.969001) (width 0.25) (layer F.Cu) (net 31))
 (segment (start 202.532999 131.158999) (end 203.708 132.334) (width 0.25) (layer B.Cu) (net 34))
 (segment (start 184.817001 131.158999) (end 202.532999 131.158999) (width 0.25) (layer B.Cu) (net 34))
 (segment (start 183.642 132.334) (end 184.817001 131.158999) (width 0.25) (layer B.Cu) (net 34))
 (segment (start 199.992999 133.509001) (end 201.168 132.334) (width 0.25) (layer F.Cu) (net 33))
 (segment (start 182.277001 133.509001) (end 199.992999 133.509001) (width 0.25) (layer F.Cu) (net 33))
 (segment (start 181.102 132.334) (end 182.277001 133.509001) (width 0.25) (layer F.Cu) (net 33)))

